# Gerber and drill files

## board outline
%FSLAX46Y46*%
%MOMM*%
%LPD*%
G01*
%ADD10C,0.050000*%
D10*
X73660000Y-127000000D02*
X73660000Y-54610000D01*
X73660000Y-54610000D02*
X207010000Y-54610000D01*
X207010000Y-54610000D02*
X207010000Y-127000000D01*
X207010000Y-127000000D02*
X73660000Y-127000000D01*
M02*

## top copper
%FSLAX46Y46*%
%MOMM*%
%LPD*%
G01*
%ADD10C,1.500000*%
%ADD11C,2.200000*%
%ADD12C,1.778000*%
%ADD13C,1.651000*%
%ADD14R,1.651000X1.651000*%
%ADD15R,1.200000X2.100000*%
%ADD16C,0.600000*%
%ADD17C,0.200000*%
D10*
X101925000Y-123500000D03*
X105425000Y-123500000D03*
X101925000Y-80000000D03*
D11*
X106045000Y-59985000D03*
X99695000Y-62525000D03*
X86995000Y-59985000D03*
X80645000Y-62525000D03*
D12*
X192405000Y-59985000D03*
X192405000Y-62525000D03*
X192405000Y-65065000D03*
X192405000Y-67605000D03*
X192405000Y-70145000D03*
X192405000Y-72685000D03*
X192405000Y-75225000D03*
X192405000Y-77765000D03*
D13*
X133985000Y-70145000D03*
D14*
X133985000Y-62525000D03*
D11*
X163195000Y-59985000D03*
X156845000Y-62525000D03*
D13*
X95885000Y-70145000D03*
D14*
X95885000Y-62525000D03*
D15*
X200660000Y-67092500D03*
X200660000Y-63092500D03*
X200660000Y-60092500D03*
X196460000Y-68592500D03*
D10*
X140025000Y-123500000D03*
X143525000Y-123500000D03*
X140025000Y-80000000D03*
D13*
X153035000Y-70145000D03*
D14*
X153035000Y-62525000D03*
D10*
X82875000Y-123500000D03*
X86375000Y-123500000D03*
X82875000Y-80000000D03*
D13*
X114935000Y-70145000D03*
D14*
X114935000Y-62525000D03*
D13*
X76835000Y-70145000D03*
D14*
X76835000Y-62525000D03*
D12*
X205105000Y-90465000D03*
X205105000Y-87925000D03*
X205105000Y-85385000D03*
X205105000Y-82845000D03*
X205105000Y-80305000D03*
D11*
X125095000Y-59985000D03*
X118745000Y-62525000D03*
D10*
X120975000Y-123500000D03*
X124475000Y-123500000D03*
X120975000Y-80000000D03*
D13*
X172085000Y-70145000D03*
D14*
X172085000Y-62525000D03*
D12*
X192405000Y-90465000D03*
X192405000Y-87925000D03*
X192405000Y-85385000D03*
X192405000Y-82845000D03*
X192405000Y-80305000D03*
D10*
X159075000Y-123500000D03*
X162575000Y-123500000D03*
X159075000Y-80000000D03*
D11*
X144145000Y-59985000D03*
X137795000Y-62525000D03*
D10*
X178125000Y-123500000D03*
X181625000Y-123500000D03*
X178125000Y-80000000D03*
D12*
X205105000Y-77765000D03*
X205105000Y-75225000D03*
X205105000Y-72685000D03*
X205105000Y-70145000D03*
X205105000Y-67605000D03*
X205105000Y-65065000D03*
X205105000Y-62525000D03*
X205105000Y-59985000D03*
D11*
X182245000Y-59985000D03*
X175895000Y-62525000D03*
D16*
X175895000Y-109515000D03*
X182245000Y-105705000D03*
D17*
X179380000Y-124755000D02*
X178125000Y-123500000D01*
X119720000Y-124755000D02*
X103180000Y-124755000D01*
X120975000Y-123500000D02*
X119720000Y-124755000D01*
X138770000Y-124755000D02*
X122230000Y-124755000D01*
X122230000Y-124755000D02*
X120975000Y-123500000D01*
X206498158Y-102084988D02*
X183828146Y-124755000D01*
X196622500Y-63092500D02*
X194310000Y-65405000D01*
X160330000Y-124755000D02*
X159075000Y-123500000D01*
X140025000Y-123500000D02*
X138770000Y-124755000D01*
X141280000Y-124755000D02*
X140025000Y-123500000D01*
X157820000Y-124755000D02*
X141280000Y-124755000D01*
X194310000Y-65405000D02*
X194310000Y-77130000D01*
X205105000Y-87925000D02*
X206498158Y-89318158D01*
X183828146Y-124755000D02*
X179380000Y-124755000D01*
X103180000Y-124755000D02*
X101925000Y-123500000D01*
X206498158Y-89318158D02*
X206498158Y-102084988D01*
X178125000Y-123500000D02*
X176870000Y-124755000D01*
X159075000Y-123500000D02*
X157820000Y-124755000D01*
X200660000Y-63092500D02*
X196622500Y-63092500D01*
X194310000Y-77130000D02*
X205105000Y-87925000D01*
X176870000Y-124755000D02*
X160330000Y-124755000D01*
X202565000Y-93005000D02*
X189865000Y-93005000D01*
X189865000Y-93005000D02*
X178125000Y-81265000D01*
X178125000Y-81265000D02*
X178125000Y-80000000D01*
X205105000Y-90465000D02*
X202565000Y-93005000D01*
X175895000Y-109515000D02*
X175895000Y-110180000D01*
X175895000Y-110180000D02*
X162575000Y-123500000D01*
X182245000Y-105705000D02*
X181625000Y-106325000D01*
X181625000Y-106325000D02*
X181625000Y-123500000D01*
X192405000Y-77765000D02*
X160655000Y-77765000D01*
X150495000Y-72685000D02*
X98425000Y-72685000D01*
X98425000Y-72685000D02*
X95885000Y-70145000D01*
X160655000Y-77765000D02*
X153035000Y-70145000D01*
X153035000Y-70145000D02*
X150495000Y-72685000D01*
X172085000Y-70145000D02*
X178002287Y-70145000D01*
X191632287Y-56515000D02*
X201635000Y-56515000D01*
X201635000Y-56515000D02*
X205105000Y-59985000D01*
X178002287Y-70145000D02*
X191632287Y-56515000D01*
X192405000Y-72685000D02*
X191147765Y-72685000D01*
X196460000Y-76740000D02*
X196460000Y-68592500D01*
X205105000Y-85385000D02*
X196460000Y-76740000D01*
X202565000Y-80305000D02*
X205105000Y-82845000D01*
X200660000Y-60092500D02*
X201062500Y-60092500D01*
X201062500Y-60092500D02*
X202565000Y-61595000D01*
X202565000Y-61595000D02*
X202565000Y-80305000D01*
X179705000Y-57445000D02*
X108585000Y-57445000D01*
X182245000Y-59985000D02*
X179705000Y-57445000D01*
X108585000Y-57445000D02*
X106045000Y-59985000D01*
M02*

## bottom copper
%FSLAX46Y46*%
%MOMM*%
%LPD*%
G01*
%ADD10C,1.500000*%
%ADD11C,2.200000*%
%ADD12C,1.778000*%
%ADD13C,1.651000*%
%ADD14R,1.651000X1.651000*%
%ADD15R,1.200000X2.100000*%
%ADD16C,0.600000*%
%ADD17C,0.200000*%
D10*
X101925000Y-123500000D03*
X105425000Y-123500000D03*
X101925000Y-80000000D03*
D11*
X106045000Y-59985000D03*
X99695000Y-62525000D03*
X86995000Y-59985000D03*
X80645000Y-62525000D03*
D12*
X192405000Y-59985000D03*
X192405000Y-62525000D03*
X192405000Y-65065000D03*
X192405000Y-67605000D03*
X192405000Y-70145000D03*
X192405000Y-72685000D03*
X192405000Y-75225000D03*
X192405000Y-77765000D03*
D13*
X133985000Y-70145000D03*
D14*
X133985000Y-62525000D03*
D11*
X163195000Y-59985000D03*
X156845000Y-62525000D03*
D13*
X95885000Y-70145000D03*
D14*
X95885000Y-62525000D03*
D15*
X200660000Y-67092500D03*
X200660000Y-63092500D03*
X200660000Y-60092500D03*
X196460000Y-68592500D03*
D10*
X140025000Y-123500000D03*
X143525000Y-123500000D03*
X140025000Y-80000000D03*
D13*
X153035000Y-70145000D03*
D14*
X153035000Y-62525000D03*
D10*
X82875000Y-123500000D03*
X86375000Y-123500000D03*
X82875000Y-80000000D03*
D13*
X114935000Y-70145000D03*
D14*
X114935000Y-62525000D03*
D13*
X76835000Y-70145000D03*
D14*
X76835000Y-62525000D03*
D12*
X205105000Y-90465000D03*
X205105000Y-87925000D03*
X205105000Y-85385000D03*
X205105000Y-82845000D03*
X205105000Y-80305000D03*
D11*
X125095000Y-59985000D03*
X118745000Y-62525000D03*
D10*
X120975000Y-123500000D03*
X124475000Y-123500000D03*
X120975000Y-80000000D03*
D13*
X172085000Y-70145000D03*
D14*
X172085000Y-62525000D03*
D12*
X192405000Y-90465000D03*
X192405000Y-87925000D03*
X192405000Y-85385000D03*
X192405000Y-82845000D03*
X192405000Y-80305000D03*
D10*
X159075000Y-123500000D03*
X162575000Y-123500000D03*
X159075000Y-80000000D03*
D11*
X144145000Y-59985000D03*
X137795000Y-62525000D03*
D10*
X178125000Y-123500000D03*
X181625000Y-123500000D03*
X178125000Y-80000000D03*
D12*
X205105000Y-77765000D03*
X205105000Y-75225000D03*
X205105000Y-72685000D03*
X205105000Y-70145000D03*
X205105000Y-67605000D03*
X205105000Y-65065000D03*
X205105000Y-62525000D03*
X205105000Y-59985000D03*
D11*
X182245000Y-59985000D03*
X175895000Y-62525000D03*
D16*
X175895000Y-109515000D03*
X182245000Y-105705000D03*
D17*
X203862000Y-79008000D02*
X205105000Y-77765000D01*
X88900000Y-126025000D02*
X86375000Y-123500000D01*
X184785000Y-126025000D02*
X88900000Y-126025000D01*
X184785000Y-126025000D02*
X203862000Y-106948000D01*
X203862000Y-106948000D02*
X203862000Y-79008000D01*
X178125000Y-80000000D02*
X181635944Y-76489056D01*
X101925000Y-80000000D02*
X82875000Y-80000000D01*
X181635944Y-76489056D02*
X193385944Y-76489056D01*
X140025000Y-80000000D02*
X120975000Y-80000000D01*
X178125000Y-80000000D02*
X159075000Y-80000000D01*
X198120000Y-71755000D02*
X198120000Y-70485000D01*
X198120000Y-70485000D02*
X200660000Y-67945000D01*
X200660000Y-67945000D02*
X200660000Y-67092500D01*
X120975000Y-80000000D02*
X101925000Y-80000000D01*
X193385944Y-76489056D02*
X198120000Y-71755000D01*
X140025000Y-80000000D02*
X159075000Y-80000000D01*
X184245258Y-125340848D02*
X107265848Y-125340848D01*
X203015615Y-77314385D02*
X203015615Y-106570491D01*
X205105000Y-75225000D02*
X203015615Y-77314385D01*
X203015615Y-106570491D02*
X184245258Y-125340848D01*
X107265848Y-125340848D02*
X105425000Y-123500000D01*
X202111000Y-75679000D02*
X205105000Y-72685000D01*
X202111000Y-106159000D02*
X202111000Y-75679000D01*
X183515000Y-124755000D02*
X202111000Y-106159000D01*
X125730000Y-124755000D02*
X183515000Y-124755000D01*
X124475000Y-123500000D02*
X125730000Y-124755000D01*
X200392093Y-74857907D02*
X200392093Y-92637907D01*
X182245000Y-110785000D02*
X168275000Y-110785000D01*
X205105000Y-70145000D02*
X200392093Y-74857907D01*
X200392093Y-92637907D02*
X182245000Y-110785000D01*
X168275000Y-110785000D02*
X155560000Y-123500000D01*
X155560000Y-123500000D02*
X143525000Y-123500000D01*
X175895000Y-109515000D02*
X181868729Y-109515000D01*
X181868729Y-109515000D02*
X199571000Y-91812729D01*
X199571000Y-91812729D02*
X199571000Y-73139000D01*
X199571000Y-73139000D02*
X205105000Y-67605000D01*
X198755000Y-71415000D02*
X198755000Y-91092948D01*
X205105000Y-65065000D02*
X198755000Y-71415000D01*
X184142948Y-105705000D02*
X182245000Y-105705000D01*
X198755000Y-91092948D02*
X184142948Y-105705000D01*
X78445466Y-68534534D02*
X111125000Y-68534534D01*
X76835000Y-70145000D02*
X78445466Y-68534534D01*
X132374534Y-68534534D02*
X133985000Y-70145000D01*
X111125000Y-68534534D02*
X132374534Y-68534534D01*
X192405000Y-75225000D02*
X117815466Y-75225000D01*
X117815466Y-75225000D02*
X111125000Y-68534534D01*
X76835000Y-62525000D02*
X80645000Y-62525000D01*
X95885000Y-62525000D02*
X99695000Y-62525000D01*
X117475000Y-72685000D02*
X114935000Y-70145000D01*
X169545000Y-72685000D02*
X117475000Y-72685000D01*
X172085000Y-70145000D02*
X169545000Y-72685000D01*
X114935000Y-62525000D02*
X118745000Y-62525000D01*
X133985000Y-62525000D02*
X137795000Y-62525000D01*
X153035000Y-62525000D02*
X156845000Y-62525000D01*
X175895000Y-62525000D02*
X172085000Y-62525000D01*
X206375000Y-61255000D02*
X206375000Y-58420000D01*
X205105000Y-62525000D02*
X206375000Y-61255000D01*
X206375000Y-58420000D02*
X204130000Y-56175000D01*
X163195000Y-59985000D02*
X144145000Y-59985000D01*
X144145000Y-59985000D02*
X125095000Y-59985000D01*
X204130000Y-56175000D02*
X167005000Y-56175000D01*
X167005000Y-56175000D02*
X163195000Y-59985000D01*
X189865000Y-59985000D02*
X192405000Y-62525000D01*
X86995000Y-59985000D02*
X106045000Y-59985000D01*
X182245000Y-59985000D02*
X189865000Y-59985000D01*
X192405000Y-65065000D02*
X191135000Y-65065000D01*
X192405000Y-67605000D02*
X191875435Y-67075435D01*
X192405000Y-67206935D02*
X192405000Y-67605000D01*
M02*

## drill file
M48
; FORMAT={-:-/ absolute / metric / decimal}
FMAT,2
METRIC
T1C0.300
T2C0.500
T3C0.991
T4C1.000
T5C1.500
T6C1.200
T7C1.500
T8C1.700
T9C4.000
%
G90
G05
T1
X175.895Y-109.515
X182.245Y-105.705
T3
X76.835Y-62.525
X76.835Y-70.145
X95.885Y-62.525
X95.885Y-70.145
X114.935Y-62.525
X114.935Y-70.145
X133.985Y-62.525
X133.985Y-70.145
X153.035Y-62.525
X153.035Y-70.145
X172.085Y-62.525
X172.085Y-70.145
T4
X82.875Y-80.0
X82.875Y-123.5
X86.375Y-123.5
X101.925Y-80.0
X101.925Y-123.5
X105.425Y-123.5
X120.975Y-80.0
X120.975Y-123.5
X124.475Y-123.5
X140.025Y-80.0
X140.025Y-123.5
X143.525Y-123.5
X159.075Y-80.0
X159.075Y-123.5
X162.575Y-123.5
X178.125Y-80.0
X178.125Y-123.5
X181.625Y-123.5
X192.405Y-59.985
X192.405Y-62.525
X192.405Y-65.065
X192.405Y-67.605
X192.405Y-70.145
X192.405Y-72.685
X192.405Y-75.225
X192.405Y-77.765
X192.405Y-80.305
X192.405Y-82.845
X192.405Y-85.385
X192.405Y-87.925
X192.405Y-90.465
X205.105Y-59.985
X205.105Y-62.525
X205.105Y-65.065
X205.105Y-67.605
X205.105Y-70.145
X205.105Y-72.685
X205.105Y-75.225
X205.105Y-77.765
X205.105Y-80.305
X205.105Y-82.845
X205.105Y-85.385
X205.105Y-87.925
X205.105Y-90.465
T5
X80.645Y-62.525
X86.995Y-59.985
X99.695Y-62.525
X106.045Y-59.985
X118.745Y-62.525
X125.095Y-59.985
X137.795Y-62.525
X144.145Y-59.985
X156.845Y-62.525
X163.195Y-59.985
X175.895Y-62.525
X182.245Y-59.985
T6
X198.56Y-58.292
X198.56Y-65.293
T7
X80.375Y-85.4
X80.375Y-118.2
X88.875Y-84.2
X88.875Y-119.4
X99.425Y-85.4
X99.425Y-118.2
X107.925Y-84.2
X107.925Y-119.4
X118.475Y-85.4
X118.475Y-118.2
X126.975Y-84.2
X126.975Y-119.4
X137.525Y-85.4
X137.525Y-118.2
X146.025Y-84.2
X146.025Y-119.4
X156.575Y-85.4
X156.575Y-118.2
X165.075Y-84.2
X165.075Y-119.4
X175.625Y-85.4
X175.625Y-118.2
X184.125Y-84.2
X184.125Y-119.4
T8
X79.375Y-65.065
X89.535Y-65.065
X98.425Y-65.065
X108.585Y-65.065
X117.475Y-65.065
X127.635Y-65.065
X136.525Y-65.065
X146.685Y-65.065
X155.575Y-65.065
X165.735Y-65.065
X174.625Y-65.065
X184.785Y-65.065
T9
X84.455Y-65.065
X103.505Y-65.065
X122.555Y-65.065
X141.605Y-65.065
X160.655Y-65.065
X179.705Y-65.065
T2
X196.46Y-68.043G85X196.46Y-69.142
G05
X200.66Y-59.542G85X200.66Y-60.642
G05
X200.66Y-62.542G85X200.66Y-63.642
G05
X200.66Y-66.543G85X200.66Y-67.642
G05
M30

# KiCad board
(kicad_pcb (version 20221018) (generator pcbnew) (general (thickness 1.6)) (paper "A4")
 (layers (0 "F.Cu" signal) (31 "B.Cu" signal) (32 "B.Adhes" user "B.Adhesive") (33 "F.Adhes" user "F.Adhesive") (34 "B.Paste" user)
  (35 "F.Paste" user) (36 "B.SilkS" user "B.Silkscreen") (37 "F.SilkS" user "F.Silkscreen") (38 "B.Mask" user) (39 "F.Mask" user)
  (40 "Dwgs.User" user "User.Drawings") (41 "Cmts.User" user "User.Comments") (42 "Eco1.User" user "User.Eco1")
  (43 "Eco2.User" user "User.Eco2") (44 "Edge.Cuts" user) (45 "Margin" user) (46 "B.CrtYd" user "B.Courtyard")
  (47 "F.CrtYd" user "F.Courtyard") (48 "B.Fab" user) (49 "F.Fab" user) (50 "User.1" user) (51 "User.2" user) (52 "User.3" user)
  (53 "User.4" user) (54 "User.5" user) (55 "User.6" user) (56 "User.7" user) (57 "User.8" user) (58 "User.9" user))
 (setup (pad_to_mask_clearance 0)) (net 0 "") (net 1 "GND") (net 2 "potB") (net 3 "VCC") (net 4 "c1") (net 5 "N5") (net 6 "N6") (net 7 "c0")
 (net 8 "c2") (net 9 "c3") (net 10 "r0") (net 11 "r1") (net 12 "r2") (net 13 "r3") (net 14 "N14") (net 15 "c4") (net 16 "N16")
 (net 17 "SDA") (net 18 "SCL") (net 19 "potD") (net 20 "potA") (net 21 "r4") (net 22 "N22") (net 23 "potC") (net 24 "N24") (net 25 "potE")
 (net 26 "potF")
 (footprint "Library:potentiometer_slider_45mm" (layer "F.Cu") (at 110.625 124.3 90)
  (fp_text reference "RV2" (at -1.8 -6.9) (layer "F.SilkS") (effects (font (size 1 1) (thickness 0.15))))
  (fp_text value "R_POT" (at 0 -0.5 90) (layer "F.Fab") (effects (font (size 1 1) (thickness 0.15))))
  (pad "" np_thru_hole circle (at 4.9 -2.7 90) (size 1.5 1.5) (drill 1.5) (layers "*.Cu" "*.Mask"))
  (pad "" np_thru_hole circle (at 6.1 -11.2 90) (size 1.5 1.5) (drill 1.5) (layers "*.Cu" "*.Mask"))
  (pad "" np_thru_hole circle (at 38.9 -11.2 90) (size 1.5 1.5) (drill 1.5) (layers "*.Cu" "*.Mask"))
  (pad "" np_thru_hole circle (at 40.1 -2.7 90) (size 1.5 1.5) (drill 1.5) (layers "*.Cu" "*.Mask"))
  (pad "1" thru_hole circle (at 0.8 -8.7 90) (size 1.5 1.5) (drill 1) (layers "*.Cu" "*.Mask") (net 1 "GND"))
  (pad "2" thru_hole circle (at 0.8 -5.2 90) (size 1.5 1.5) (drill 1) (layers "*.Cu" "*.Mask") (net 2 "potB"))
  (pad "3" thru_hole circle (at 44.3 -8.7 90) (size 1.5 1.5) (drill 1) (layers "*.Cu" "*.Mask") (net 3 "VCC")))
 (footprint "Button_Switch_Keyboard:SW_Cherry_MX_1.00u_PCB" (layer "F.Cu") (at 106.045 59.985)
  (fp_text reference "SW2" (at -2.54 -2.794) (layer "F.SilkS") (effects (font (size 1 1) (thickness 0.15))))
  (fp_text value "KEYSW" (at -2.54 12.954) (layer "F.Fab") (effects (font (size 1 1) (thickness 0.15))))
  (pad "" np_thru_hole circle (at -7.62 5.08) (size 1.7 1.7) (drill 1.7) (layers "*.Cu" "*.Mask"))
  (pad "" np_thru_hole circle (at -2.54 5.08) (size 4 4) (drill 4) (layers "*.Cu" "*.Mask"))
  (pad "" np_thru_hole circle (at 2.54 5.08) (size 1.7 1.7) (drill 1.7) (layers "*.Cu" "*.Mask"))
  (pad "1" thru_hole circle (at 0 0) (size 2.2 2.2) (drill 1.5) (layers "*.Cu" "*.Mask") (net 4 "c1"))
  (pad "2" thru_hole circle (at -6.35 2.54) (size 2.2 2.2) (drill 1.5) (layers "*.Cu" "*.Mask") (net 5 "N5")))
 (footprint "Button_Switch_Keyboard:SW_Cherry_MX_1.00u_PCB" (layer "F.Cu") (at 86.995 59.985)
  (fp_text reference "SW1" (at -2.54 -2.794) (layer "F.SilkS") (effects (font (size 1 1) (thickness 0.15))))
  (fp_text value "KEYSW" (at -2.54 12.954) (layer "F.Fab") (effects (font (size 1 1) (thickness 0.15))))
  (pad "" np_thru_hole circle (at -7.62 5.08) (size 1.7 1.7) (drill 1.7) (layers "*.Cu" "*.Mask"))
  (pad "" np_thru_hole circle (at -2.54 5.08) (size 4 4) (drill 4) (layers "*.Cu" "*.Mask"))
  (pad "" np_thru_hole circle (at 2.54 5.08) (size 1.7 1.7) (drill 1.7) (layers "*.Cu" "*.Mask"))
  (pad "1" thru_hole circle (at 0 0) (size 2.2 2.2) (drill 1.5) (layers "*.Cu" "*.Mask") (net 4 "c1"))
  (pad "2" thru_hole circle (at -6.35 2.54) (size 2.2 2.2) (drill 1.5) (layers "*.Cu" "*.Mask") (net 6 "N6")))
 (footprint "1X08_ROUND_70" (layer "F.Cu") (at 192.405 68.875 -90)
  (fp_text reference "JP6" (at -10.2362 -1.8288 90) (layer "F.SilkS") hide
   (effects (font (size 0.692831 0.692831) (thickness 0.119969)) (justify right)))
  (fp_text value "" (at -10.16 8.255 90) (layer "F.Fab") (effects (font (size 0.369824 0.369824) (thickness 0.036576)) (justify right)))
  (pad "1" thru_hole circle (at -8.89 0) (size 1.778 1.778) (drill 1) (layers "*.Cu" "*.Mask") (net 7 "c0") (solder_mask_margin 0.0508))
  (pad "2" thru_hole circle (at -6.35 0) (size 1.778 1.778) (drill 1) (layers "*.Cu" "*.Mask") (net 4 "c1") (solder_mask_margin 0.0508))
  (pad "3" thru_hole circle (at -3.81 0) (size 1.778 1.778) (drill 1) (layers "*.Cu" "*.Mask") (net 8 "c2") (solder_mask_margin 0.0508))
  (pad "4" thru_hole circle (at -1.27 0) (size 1.778 1.778) (drill 1) (layers "*.Cu" "*.Mask") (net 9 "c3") (solder_mask_margin 0.0508))
  (pad "5" thru_hole circle (at 1.27 0) (size 1.778 1.778) (drill 1) (layers "*.Cu" "*.Mask") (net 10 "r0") (solder_mask_margin 0.0508))
  (pad "6" thru_hole circle (at 3.81 0) (size 1.778 1.778) (drill 1) (layers "*.Cu" "*.Mask") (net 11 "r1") (solder_mask_margin 0.0508))
  (pad "7" thru_hole circle (at 6.35 0) (size 1.778 1.778) (drill 1) (layers "*.Cu" "*.Mask") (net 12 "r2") (solder_mask_margin 0.0508))
  (pad "8" thru_hole circle (at 8.89 0) (size 1.778 1.778) (drill 1) (layers "*.Cu" "*.Mask") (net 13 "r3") (solder_mask_margin 0.0508)))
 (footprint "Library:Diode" (layer "F.Cu") (at 133.985 66.335 90)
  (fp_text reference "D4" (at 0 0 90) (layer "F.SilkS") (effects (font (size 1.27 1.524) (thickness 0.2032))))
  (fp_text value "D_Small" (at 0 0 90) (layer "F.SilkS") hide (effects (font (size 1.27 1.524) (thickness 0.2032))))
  (pad "1" thru_hole circle (at -3.81 0 90) (size 1.651 1.651) (drill 0.9906) (layers "*.Cu" "*.SilkS" "*.Mask") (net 12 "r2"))
  (pad "2" thru_hole rect (at 3.81 0 90) (size 1.651 1.651) (drill 0.9906) (layers "*.Cu" "*.SilkS" "*.Mask") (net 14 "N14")))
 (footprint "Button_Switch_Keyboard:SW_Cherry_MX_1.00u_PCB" (layer "F.Cu") (at 163.195 59.985)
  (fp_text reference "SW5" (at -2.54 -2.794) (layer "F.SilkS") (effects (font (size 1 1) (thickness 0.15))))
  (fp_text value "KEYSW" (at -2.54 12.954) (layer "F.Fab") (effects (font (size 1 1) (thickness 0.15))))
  (pad "" np_thru_hole circle (at -7.62 5.08) (size 1.7 1.7) (drill 1.7) (layers "*.Cu" "*.Mask"))
  (pad "" np_thru_hole circle (at -2.54 5.08) (size 4 4) (drill 4) (layers "*.Cu" "*.Mask"))
  (pad "" np_thru_hole circle (at 2.54 5.08) (size 1.7 1.7) (drill 1.7) (layers "*.Cu" "*.Mask"))
  (pad "1" thru_hole circle (at 0 0) (size 2.2 2.2) (drill 1.5) (layers "*.Cu" "*.Mask") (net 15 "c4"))
  (pad "2" thru_hole circle (at -6.35 2.54) (size 2.2 2.2) (drill 1.5) (layers "*.Cu" "*.Mask") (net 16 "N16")))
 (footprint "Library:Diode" (layer "F.Cu") (at 95.885 66.335 90)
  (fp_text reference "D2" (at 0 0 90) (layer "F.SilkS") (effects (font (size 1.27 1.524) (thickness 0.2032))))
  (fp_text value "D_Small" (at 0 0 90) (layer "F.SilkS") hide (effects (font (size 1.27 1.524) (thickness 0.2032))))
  (pad "1" thru_hole circle (at -3.81 0 90) (size 1.651 1.651) (drill 0.9906) (layers "*.Cu" "*.SilkS" "*.Mask") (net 13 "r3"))
  (pad "2" thru_hole rect (at 3.81 0 90) (size 1.651 1.651) (drill 0.9906) (layers "*.Cu" "*.SilkS" "*.Mask") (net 5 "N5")))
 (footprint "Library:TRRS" (layer "F.Cu") (at 198.56 56.7925)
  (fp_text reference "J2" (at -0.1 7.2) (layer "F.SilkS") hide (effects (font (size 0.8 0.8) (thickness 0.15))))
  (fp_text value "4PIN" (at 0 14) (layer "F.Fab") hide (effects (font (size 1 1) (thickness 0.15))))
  (pad "" np_thru_hole circle (at 0 1.5) (size 1.2 1.2) (drill 1.2) (layers "*.Cu" "*.Mask" "F.SilkS"))
  (pad "" np_thru_hole circle (at 0 8.5) (size 1.2 1.2) (drill 1.2) (layers "*.Cu" "*.Mask" "F.SilkS"))
  (pad "1" thru_hole rect (at 2.1 10.3) (size 1.2 2.1) (drill oval 0.5 1.6) (layers "*.Cu" "*.Mask" "F.SilkS") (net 3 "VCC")
   (clearance 0.15))
  (pad "2" thru_hole rect (at 2.1 6.3) (size 1.2 2.1) (drill oval 0.5 1.6) (layers "*.Cu" "*.Mask" "F.SilkS") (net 1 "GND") (clearance 0.15))
  (pad "3" thru_hole rect (at 2.1 3.3) (size 1.2 2.1) (drill oval 0.5 1.6) (layers "*.Cu" "*.Mask" "F.SilkS") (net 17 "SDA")
   (clearance 0.15))
  (pad "4" thru_hole rect (at -2.1 11.8) (size 1.2 2.1) (drill oval 0.5 1.6) (layers "*.Cu" "*.Mask" "F.SilkS") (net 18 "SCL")
   (clearance 0.15)))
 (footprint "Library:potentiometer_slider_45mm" (layer "F.Cu") (at 148.725 124.3 90)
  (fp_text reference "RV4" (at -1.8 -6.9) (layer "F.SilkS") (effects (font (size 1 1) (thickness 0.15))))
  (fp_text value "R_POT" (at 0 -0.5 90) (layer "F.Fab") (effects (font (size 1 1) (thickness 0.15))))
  (pad "" np_thru_hole circle (at 4.9 -2.7 90) (size 1.5 1.5) (drill 1.5) (layers "*.Cu" "*.Mask"))
  (pad "" np_thru_hole circle (at 6.1 -11.2 90) (size 1.5 1.5) (drill 1.5) (layers "*.Cu" "*.Mask"))
  (pad "" np_thru_hole circle (at 38.9 -11.2 90) (size 1.5 1.5) (drill 1.5) (layers "*.Cu" "*.Mask"))
  (pad "" np_thru_hole circle (at 40.1 -2.7 90) (size 1.5 1.5) (drill 1.5) (layers "*.Cu" "*.Mask"))
  (pad "1" thru_hole circle (at 0.8 -8.7 90) (size 1.5 1.5) (drill 1) (layers "*.Cu" "*.Mask") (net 1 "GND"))
  (pad "2" thru_hole circle (at 0.8 -5.2 90) (size 1.5 1.5) (drill 1) (layers "*.Cu" "*.Mask") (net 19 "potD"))
  (pad "3" thru_hole circle (at 44.3 -8.7 90) (size 1.5 1.5) (drill 1) (layers "*.Cu" "*.Mask") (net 3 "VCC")))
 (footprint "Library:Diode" (layer "F.Cu") (at 153.035 66.335 90)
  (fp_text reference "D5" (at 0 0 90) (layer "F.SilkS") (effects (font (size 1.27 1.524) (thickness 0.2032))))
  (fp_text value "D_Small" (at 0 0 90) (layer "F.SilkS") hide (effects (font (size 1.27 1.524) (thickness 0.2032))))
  (pad "1" thru_hole circle (at -3.81 0 90) (size 1.651 1.651) (drill 0.9906) (layers "*.Cu" "*.SilkS" "*.Mask") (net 13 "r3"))
  (pad "2" thru_hole rect (at 3.81 0 90) (size 1.651 1.651) (drill 0.9906) (layers "*.Cu" "*.SilkS" "*.Mask") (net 16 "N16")))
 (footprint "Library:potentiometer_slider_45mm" (layer "F.Cu") (at 91.575 124.3 90)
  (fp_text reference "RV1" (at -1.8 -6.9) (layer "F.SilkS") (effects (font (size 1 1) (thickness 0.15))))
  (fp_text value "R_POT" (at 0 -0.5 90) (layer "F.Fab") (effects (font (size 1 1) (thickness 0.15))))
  (pad "" np_thru_hole circle (at 4.9 -2.7 90) (size 1.5 1.5) (drill 1.5) (layers "*.Cu" "*.Mask"))
  (pad "" np_thru_hole circle (at 6.1 -11.2 90) (size 1.5 1.5) (drill 1.5) (layers "*.Cu" "*.Mask"))
  (pad "" np_thru_hole circle (at 38.9 -11.2 90) (size 1.5 1.5) (drill 1.5) (layers "*.Cu" "*.Mask"))
  (pad "" np_thru_hole circle (at 40.1 -2.7 90) (size 1.5 1.5) (drill 1.5) (layers "*.Cu" "*.Mask"))
  (pad "1" thru_hole circle (at 0.8 -8.7 90) (size 1.5 1.5) (drill 1) (layers "*.Cu" "*.Mask") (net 1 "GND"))
  (pad "2" thru_hole circle (at 0.8 -5.2 90) (size 1.5 1.5) (drill 1) (layers "*.Cu" "*.Mask") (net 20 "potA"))
  (pad "3" thru_hole circle (at 44.3 -8.7 90) (size 1.5 1.5) (drill 1) (layers "*.Cu" "*.Mask") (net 3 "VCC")))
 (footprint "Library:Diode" (layer "F.Cu") (at 114.935 66.335 90)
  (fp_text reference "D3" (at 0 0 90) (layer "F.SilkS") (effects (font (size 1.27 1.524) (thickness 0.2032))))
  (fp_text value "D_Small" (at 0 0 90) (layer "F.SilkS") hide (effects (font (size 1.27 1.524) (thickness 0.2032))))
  (pad "1" thru_hole circle (at -3.81 0 90) (size 1.651 1.651) (drill 0.9906) (layers "*.Cu" "*.SilkS" "*.Mask") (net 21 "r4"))
  (pad "2" thru_hole rect (at 3.81 0 90) (size 1.651 1.651) (drill 0.9906) (layers "*.Cu" "*.SilkS" "*.Mask") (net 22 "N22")))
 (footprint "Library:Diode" (layer "F.Cu") (at 76.835 66.335 90)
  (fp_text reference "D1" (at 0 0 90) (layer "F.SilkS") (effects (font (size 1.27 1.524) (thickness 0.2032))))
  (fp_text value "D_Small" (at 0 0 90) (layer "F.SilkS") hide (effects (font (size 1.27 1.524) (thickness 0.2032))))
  (pad "1" thru_hole circle (at -3.81 0 90) (size 1.651 1.651) (drill 0.9906) (layers "*.Cu" "*.SilkS" "*.Mask") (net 12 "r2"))
  (pad "2" thru_hole rect (at 3.81 0 90) (size 1.651 1.651) (drill 0.9906) (layers "*.Cu" "*.SilkS" "*.Mask") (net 6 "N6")))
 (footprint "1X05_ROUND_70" (layer "F.Cu") (at 205.105 85.385 90)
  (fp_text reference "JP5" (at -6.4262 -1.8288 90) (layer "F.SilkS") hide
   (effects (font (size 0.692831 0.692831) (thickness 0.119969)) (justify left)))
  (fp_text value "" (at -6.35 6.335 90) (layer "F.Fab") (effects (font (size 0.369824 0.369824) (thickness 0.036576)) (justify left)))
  (pad "1" thru_hole circle (at -5.08 0 180) (size 1.778 1.778) (drill 1) (layers "*.Cu" "*.Mask") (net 3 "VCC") (solder_mask_margin 0.0508))
  (pad "2" thru_hole circle (at -2.54 0 180) (size 1.778 1.778) (drill 1) (layers "*.Cu" "*.Mask") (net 1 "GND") (solder_mask_margin 0.0508))
  (pad "3" thru_hole circle (at 0 0 180) (size 1.778 1.778) (drill 1) (layers "*.Cu" "*.Mask") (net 18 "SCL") (solder_mask_margin 0.0508))
  (pad "4" thru_hole circle (at 2.54 0 180) (size 1.778 1.778) (drill 1) (layers "*.Cu" "*.Mask") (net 17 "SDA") (solder_mask_margin 0.0508))
  (pad "5" thru_hole circle (at 5.08 0 180) (size 1.778 1.778) (drill 1) (layers "*.Cu" "*.Mask") (solder_mask_margin 0.0508)))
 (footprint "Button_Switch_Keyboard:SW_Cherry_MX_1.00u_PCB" (layer "F.Cu") (at 125.095 59.985)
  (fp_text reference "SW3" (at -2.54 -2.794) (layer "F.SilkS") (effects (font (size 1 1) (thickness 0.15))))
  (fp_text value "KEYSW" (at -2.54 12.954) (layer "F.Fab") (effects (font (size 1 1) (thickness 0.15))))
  (pad "" np_thru_hole circle (at -7.62 5.08) (size 1.7 1.7) (drill 1.7) (layers "*.Cu" "*.Mask"))
  (pad "" np_thru_hole circle (at -2.54 5.08) (size 4 4) (drill 4) (layers "*.Cu" "*.Mask"))
  (pad "" np_thru_hole circle (at 2.54 5.08) (size 1.7 1.7) (drill 1.7) (layers "*.Cu" "*.Mask"))
  (pad "1" thru_hole circle (at 0 0) (size 2.2 2.2) (drill 1.5) (layers "*.Cu" "*.Mask") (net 15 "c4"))
  (pad "2" thru_hole circle (at -6.35 2.54) (size 2.2 2.2) (drill 1.5) (layers "*.Cu" "*.Mask") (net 22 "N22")))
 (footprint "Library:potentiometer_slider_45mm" (layer "F.Cu") (at 129.675 124.3 90)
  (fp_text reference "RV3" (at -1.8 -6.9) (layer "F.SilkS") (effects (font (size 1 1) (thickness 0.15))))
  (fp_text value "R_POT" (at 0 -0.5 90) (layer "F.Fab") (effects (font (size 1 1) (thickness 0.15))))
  (pad "" np_thru_hole circle (at 4.9 -2.7 90) (size 1.5 1.5) (drill 1.5) (layers "*.Cu" "*.Mask"))
  (pad "" np_thru_hole circle (at 6.1 -11.2 90) (size 1.5 1.5) (drill 1.5) (layers "*.Cu" "*.Mask"))
  (pad "" np_thru_hole circle (at 38.9 -11.2 90) (size 1.5 1.5) (drill 1.5) (layers "*.Cu" "*.Mask"))
  (pad "" np_thru_hole circle (at 40.1 -2.7 90) (size 1.5 1.5) (drill 1.5) (layers "*.Cu" "*.Mask"))
  (pad "1" thru_hole circle (at 0.8 -8.7 90) (size 1.5 1.5) (drill 1) (layers "*.Cu" "*.Mask") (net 1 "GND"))
  (pad "2" thru_hole circle (at 0.8 -5.2 90) (size 1.5 1.5) (drill 1) (layers "*.Cu" "*.Mask") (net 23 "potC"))
  (pad "3" thru_hole circle (at 44.3 -8.7 90) (size 1.5 1.5) (drill 1) (layers "*.Cu" "*.Mask") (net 3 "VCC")))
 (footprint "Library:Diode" (layer "F.Cu") (at 172.085 66.335 90)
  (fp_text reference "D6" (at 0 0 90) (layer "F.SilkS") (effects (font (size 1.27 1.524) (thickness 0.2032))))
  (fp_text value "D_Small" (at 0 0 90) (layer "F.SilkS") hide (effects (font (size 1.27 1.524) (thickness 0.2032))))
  (pad "1" thru_hole circle (at -3.81 0 90) (size 1.651 1.651) (drill 0.9906) (layers "*.Cu" "*.SilkS" "*.Mask") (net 21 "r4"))
  (pad "2" thru_hole rect (at 3.81 0 90) (size 1.651 1.651) (drill 0.9906) (layers "*.Cu" "*.SilkS" "*.Mask") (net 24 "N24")))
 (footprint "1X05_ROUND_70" (layer "F.Cu") (at 192.405 85.385 90)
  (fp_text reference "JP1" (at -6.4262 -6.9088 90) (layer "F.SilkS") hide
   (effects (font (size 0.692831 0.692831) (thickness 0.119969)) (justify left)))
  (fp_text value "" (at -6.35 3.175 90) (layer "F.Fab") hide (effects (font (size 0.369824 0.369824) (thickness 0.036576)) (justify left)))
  (pad "1" thru_hole circle (at -5.08 0 180) (size 1.778 1.778) (drill 1) (layers "*.Cu" "*.Mask") (solder_mask_margin 0.0508))
  (pad "2" thru_hole circle (at -2.54 0 180) (size 1.778 1.778) (drill 1) (layers "*.Cu" "*.Mask") (solder_mask_margin 0.0508))
  (pad "3" thru_hole circle (at 0 0 180) (size 1.778 1.778) (drill 1) (layers "*.Cu" "*.Mask") (solder_mask_margin 0.0508))
  (pad "4" thru_hole circle (at 2.54 0 180) (size 1.778 1.778) (drill 1) (layers "*.Cu" "*.Mask") (solder_mask_margin 0.0508))
  (pad "5" thru_hole circle (at 5.08 0 180) (size 1.778 1.778) (drill 1) (layers "*.Cu" "*.Mask") (solder_mask_margin 0.0508)))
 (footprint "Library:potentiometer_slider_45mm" (layer "F.Cu") (at 167.775 124.3 90)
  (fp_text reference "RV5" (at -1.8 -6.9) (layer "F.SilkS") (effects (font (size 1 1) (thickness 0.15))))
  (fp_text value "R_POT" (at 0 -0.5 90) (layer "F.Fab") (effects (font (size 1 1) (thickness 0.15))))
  (pad "" np_thru_hole circle (at 4.9 -2.7 90) (size 1.5 1.5) (drill 1.5) (layers "*.Cu" "*.Mask"))
  (pad "" np_thru_hole circle (at 6.1 -11.2 90) (size 1.5 1.5) (drill 1.5) (layers "*.Cu" "*.Mask"))
  (pad "" np_thru_hole circle (at 38.9 -11.2 90) (size 1.5 1.5) (drill 1.5) (layers "*.Cu" "*.Mask"))
  (pad "" np_thru_hole circle (at 40.1 -2.7 90) (size 1.5 1.5) (drill 1.5) (layers "*.Cu" "*.Mask"))
  (pad "1" thru_hole circle (at 0.8 -8.7 90) (size 1.5 1.5) (drill 1) (layers "*.Cu" "*.Mask") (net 1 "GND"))
  (pad "2" thru_hole circle (at 0.8 -5.2 90) (size 1.5 1.5) (drill 1) (layers "*.Cu" "*.Mask") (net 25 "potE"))
  (pad "3" thru_hole circle (at 44.3 -8.7 90) (size 1.5 1.5) (drill 1) (layers "*.Cu" "*.Mask") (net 3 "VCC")))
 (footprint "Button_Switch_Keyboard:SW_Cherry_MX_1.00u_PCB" (layer "F.Cu") (at 144.145 59.985)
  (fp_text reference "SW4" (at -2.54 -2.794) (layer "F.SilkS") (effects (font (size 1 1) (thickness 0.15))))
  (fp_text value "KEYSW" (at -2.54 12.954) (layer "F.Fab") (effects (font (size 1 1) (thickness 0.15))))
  (pad "" np_thru_hole circle (at -7.62 5.08) (size 1.7 1.7) (drill 1.7) (layers "*.Cu" "*.Mask"))
  (pad "" np_thru_hole circle (at -2.54 5.08) (size 4 4) (drill 4) (layers "*.Cu" "*.Mask"))
  (pad "" np_thru_hole circle (at 2.54 5.08) (size 1.7 1.7) (drill 1.7) (layers "*.Cu" "*.Mask"))
  (pad "1" thru_hole circle (at 0 0) (size 2.2 2.2) (drill 1.5) (layers "*.Cu" "*.Mask") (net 15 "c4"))
  (pad "2" thru_hole circle (at -6.35 2.54) (size 2.2 2.2) (drill 1.5) (layers "*.Cu" "*.Mask") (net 14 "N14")))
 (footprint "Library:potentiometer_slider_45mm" (layer "F.Cu") (at 186.825 124.3 90)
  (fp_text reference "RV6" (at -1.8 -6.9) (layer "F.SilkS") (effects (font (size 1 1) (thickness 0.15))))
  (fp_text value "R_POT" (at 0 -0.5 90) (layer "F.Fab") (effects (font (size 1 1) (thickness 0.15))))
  (pad "" np_thru_hole circle (at 4.9 -2.7 90) (size 1.5 1.5) (drill 1.5) (layers "*.Cu" "*.Mask"))
  (pad "" np_thru_hole circle (at 6.1 -11.2 90) (size 1.5 1.5) (drill 1.5) (layers "*.Cu" "*.Mask"))
  (pad "" np_thru_hole circle (at 38.9 -11.2 90) (size 1.5 1.5) (drill 1.5) (layers "*.Cu" "*.Mask"))
  (pad "" np_thru_hole circle (at 40.1 -2.7 90) (size 1.5 1.5) (drill 1.5) (layers "*.Cu" "*.Mask"))
  (pad "1" thru_hole circle (at 0.8 -8.7 90) (size 1.5 1.5) (drill 1) (layers "*.Cu" "*.Mask") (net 1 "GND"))
  (pad "2" thru_hole circle (at 0.8 -5.2 90) (size 1.5 1.5) (drill 1) (layers "*.Cu" "*.Mask") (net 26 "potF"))
  (pad "3" thru_hole circle (at 44.3 -8.7 90) (size 1.5 1.5) (drill 1) (layers "*.Cu" "*.Mask") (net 3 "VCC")))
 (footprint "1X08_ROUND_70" (layer "F.Cu") (at 205.105 68.875 90)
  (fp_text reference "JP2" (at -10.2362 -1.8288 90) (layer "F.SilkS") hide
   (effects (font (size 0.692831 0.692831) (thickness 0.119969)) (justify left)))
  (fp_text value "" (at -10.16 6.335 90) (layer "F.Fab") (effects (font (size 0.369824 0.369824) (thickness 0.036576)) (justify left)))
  (pad "1" thru_hole circle (at -8.89 0 180) (size 1.778 1.778) (drill 1) (layers "*.Cu" "*.Mask") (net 20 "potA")
   (solder_mask_margin 0.0508))
  (pad "2" thru_hole circle (at -6.35 0 180) (size 1.778 1.778) (drill 1) (layers "*.Cu" "*.Mask") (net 2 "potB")
   (solder_mask_margin 0.0508))
  (pad "3" thru_hole circle (at -3.81 0 180) (size 1.778 1.778) (drill 1) (layers "*.Cu" "*.Mask") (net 23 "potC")
   (solder_mask_margin 0.0508))
  (pad "4" thru_hole circle (at -1.27 0 180) (size 1.778 1.778) (drill 1) (layers "*.Cu" "*.Mask") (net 19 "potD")
   (solder_mask_margin 0.0508))
  (pad "5" thru_hole circle (at 1.27 0 180) (size 1.778 1.778) (drill 1) (layers "*.Cu" "*.Mask") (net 25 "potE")
   (solder_mask_margin 0.0508))
  (pad "6" thru_hole circle (at 3.81 0 180) (size 1.778 1.778) (drill 1) (layers "*.Cu" "*.Mask") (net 26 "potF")
   (solder_mask_margin 0.0508))
  (pad "7" thru_hole circle (at 6.35 0 180) (size 1.778 1.778) (drill 1) (layers "*.Cu" "*.Mask") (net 15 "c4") (solder_mask_margin 0.0508))
  (pad "8" thru_hole circle (at 8.89 0 180) (size 1.778 1.778) (drill 1) (layers "*.Cu" "*.Mask") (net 21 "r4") (solder_mask_margin 0.0508)))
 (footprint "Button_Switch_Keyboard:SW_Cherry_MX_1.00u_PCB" (layer "F.Cu") (at 182.245 59.985)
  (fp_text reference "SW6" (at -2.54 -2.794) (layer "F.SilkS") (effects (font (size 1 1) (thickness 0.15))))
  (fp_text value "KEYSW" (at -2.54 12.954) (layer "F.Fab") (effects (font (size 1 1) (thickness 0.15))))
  (pad "" np_thru_hole circle (at -7.62 5.08) (size 1.7 1.7) (drill 1.7) (layers "*.Cu" "*.Mask"))
  (pad "" np_thru_hole circle (at -2.54 5.08) (size 4 4) (drill 4) (layers "*.Cu" "*.Mask"))
  (pad "" np_thru_hole circle (at 2.54 5.08) (size 1.7 1.7) (drill 1.7) (layers "*.Cu" "*.Mask"))
  (pad "1" thru_hole circle (at 0 0) (size 2.2 2.2) (drill 1.5) (layers "*.Cu" "*.Mask") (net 4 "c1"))
  (pad "2" thru_hole circle (at -6.35 2.54) (size 2.2 2.2) (drill 1.5) (layers "*.Cu" "*.Mask") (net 24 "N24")))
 (gr_line (start 73.66 127) (end 73.66 54.61) (stroke (width 0.05) (type default)) (layer "Edge.Cuts"))
 (gr_line (start 73.66 54.61) (end 207.01 54.61) (stroke (width 0.05) (type default)) (layer "Edge.Cuts"))
 (gr_line (start 207.01 54.61) (end 207.01 127) (stroke (width 0.05) (type default)) (layer "Edge.Cuts"))
 (gr_line (start 207.01 127) (end 73.66 127) (stroke (width 0.05) (type default)) (layer "Edge.Cuts"))
 (segment (start 179.38 124.755) (end 178.125 123.5) (width 0.2) (layer "F.Cu") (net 1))
 (segment (start 119.72 124.755) (end 103.18 124.755) (width 0.2) (layer "F.Cu") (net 1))
 (segment (start 120.975 123.5) (end 119.72 124.755) (width 0.2) (layer "F.Cu") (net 1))
 (segment (start 138.77 124.755) (end 122.23 124.755) (width 0.2) (layer "F.Cu") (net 1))
 (segment (start 122.23 124.755) (end 120.975 123.5) (width 0.2) (layer "F.Cu") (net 1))
 (segment (start 206.498158 102.084988) (end 183.828146 124.755) (width 0.2) (layer "F.Cu") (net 1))
 (segment (start 196.6225 63.0925) (end 194.31 65.405) (width 0.2) (layer "F.Cu") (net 1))
 (segment (start 160.33 124.755) (end 159.075 123.5) (width 0.2) (layer "F.Cu") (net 1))
 (segment (start 140.025 123.5) (end 138.77 124.755) (width 0.2) (layer "F.Cu") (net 1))
 (segment (start 141.28 124.755) (end 140.025 123.5) (width 0.2) (layer "F.Cu") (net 1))
 (segment (start 157.82 124.755) (end 141.28 124.755) (width 0.2) (layer "F.Cu") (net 1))
 (segment (start 194.31 65.405) (end 194.31 77.13) (width 0.2) (layer "F.Cu") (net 1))
 (segment (start 205.105 87.925) (end 206.498158 89.318158) (width 0.2) (layer "F.Cu") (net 1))
 (segment (start 183.828146 124.755) (end 179.38 124.755) (width 0.2) (layer "F.Cu") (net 1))
 (segment (start 103.18 124.755) (end 101.925 123.5) (width 0.2) (layer "F.Cu") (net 1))
 (segment (start 206.498158 89.318158) (end 206.498158 102.084988) (width 0.2) (layer "F.Cu") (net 1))
 (segment (start 178.125 123.5) (end 176.87 124.755) (width 0.2) (layer "F.Cu") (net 1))
 (segment (start 159.075 123.5) (end 157.82 124.755) (width 0.2) (layer "F.Cu") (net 1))
 (segment (start 200.66 63.0925) (end 196.6225 63.0925) (width 0.2) (layer "F.Cu") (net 1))
 (segment (start 194.31 77.13) (end 205.105 87.925) (width 0.2) (layer "F.Cu") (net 1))
 (segment (start 176.87 124.755) (end 160.33 124.755) (width 0.2) (layer "F.Cu") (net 1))
 (segment (start 203.862 79.008) (end 205.105 77.765) (width 0.2) (layer "B.Cu") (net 20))
 (segment (start 88.9 126.025) (end 86.375 123.5) (width 0.2) (layer "B.Cu") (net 20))
 (segment (start 184.785 126.025) (end 88.9 126.025) (width 0.2) (layer "B.Cu") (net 20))
 (segment (start 184.785 126.025) (end 203.862 106.948) (width 0.2) (layer "B.Cu") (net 20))
 (segment (start 203.862 106.948) (end 203.862 79.008) (width 0.2) (layer "B.Cu") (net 20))
 (segment (start 202.565 93.005) (end 189.865 93.005) (width 0.2) (layer "F.Cu") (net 3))
 (segment (start 189.865 93.005) (end 178.125 81.265) (width 0.2) (layer "F.Cu") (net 3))
 (segment (start 178.125 81.265) (end 178.125 80) (width 0.2) (layer "F.Cu") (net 3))
 (segment (start 205.105 90.465) (end 202.565 93.005) (width 0.2) (layer "F.Cu") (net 3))
 (segment (start 178.125 80) (end 181.635944 76.489056) (width 0.2) (layer "B.Cu") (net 3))
 (segment (start 101.925 80) (end 82.875 80) (width 0.2) (layer "B.Cu") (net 3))
 (segment (start 181.635944 76.489056) (end 193.385944 76.489056) (width 0.2) (layer "B.Cu") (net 3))
 (segment (start 140.025 80) (end 120.975 80) (width 0.2) (layer "B.Cu") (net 3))
 (segment (start 178.125 80) (end 159.075 80) (width 0.2) (layer "B.Cu") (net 3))
 (segment (start 198.12 71.755) (end 198.12 70.485) (width 0.2) (layer "B.Cu") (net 3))
 (segment (start 198.12 70.485) (end 200.66 67.945) (width 0.2) (layer "B.Cu") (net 3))
 (segment (start 200.66 67.945) (end 200.66 67.0925) (width 0.2) (layer "B.Cu") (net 3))
 (segment (start 120.975 80) (end 101.925 80) (width 0.2) (layer "B.Cu") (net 3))
 (segment (start 193.385944 76.489056) (end 198.12 71.755) (width 0.2) (layer "B.Cu") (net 3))
 (segment (start 140.025 80) (end 159.075 80) (width 0.2) (layer "B.Cu") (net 3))
 (segment (start 184.245258 125.340848) (end 107.265848 125.340848) (width 0.2) (layer "B.Cu") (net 2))
 (segment (start 203.015615 77.314385) (end 203.015615 106.570491) (width 0.2) (layer "B.Cu") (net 2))
 (segment (start 205.105 75.225) (end 203.015615 77.314385) (width 0.2) (layer "B.Cu") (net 2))
 (segment (start 203.015615 106.570491) (end 184.245258 125.340848) (width 0.2) (layer "B.Cu") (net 2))
 (segment (start 107.265848 125.340848) (end 105.425 123.5) (width 0.2) (layer "B.Cu") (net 2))
 (segment (start 202.111 75.679) (end 205.105 72.685) (width 0.2) (layer "B.Cu") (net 23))
 (segment (start 202.111 106.159) (end 202.111 75.679) (width 0.2) (layer "B.Cu") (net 23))
 (segment (start 183.515 124.755) (end 202.111 106.159) (width 0.2) (layer "B.Cu") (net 23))
 (segment (start 125.73 124.755) (end 183.515 124.755) (width 0.2) (layer "B.Cu") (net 23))
 (segment (start 124.475 123.5) (end 125.73 124.755) (width 0.2) (layer "B.Cu") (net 23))
 (segment (start 200.392093 74.857907) (end 200.392093 92.637907) (width 0.2) (layer "B.Cu") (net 19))
 (segment (start 182.245 110.785) (end 168.275 110.785) (width 0.2) (layer "B.Cu") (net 19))
 (segment (start 205.105 70.145) (end 200.392093 74.857907) (width 0.2) (layer "B.Cu") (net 19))
 (segment (start 200.392093 92.637907) (end 182.245 110.785) (width 0.2) (layer "B.Cu") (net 19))
 (segment (start 168.275 110.785) (end 155.56 123.5) (width 0.2) (layer "B.Cu") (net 19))
 (segment (start 155.56 123.5) (end 143.525 123.5) (width 0.2) (layer "B.Cu") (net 19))
 (segment (start 175.895 109.515) (end 175.895 110.18) (width 0.2) (layer "F.Cu") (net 25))
 (segment (start 175.895 110.18) (end 162.575 123.5) (width 0.2) (layer "F.Cu") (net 25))
 (via (at 175.895 109.515) (size 0.6) (drill 0.3) (layers "F.Cu" "B.Cu") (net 25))
 (segment (start 175.895 109.515) (end 181.868729 109.515) (width 0.2) (layer "B.Cu") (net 25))
 (segment (start 181.868729 109.515) (end 199.571 91.812729) (width 0.2) (layer "B.Cu") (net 25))
 (segment (start 199.571 91.812729) (end 199.571 73.139) (width 0.2) (layer "B.Cu") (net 25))
 (segment (start 199.571 73.139) (end 205.105 67.605) (width 0.2) (layer "B.Cu") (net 25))
 (segment (start 182.245 105.705) (end 181.625 106.325) (width 0.2) (layer "F.Cu") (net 26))
 (segment (start 181.625 106.325) (end 181.625 123.5) (width 0.2) (layer "F.Cu") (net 26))
 (via (at 182.245 105.705) (size 0.6) (drill 0.3) (layers "F.Cu" "B.Cu") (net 26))
 (segment (start 198.755 71.415) (end 198.755 91.092948) (width 0.2) (layer "B.Cu") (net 26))
 (segment (start 205.105 65.065) (end 198.755 71.415) (width 0.2) (layer "B.Cu") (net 26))
 (segment (start 184.142948 105.705) (end 182.245 105.705) (width 0.2) (layer "B.Cu") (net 26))
 (segment (start 198.755 91.092948) (end 184.142948 105.705) (width 0.2) (layer "B.Cu") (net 26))
 (segment (start 78.445466 68.534534) (end 111.125 68.534534) (width 0.2) (layer "B.Cu") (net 12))
 (segment (start 76.835 70.145) (end 78.445466 68.534534) (width 0.2) (layer "B.Cu") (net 12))
 (segment (start 132.374534 68.534534) (end 133.985 70.145) (width 0.2) (layer "B.Cu") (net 12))
 (segment (start 111.125 68.534534) (end 132.374534 68.534534) (width 0.2) (layer "B.Cu") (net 12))
 (segment (start 192.405 75.225) (end 117.815466 75.225) (width 0.2) (layer "B.Cu") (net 12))
 (segment (start 117.815466 75.225) (end 111.125 68.534534) (width 0.2) (layer "B.Cu") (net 12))
 (segment (start 76.835 62.525) (end 80.645 62.525) (width 0.2) (layer "B.Cu") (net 6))
 (segment (start 192.405 77.765) (end 160.655 77.765) (width 0.2) (layer "F.Cu") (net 13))
 (segment (start 150.495 72.685) (end 98.425 72.685) (width 0.2) (layer "F.Cu") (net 13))
 (segment (start 98.425 72.685) (end 95.885 70.145) (width 0.2) (layer "F.Cu") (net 13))
 (segment (start 160.655 77.765) (end 153.035 70.145) (width 0.2) (layer "F.Cu") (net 13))
 (segment (start 153.035 70.145) (end 150.495 72.685) (width 0.2) (layer "F.Cu") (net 13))
 (segment (start 95.885 62.525) (end 99.695 62.525) (width 0.2) (layer "B.Cu") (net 5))
 (segment (start 172.085 70.145) (end 178.002287 70.145) (width 0.2) (layer "F.Cu") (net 21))
 (segment (start 191.632287 56.515) (end 201.635 56.515) (width 0.2) (layer "F.Cu") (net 21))
 (segment (start 201.635 56.515) (end 205.105 59.985) (width 0.2) (layer "F.Cu") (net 21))
 (segment (start 178.002287 70.145) (end 191.632287 56.515) (width 0.2) (layer "F.Cu") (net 21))
 (segment (start 117.475 72.685) (end 114.935 70.145) (width 0.2) (layer "B.Cu") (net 21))
 (segment (start 169.545 72.685) (end 117.475 72.685) (width 0.2) (layer "B.Cu") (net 21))
 (segment (start 172.085 70.145) (end 169.545 72.685) (width 0.2) (layer "B.Cu") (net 21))
 (segment (start 114.935 62.525) (end 118.745 62.525) (width 0.2) (layer "B.Cu") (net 22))
 (segment (start 133.985 62.525) (end 137.795 62.525) (width 0.2) (layer "B.Cu") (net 14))
 (segment (start 153.035 62.525) (end 156.845 62.525) (width 0.2) (layer "B.Cu") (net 16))
 (segment (start 175.895 62.525) (end 172.085 62.525) (width 0.2) (layer "B.Cu") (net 24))
 (segment (start 192.405 72.685) (end 191.147765 72.685) (width 0.2) (layer "F.Cu") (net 11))
 (segment (start 196.46 76.74) (end 196.46 68.5925) (width 0.2) (layer "F.Cu") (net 18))
 (segment (start 205.105 85.385) (end 196.46 76.74) (width 0.2) (layer "F.Cu") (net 18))
 (segment (start 202.565 80.305) (end 205.105 82.845) (width 0.2) (layer "F.Cu") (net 17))
 (segment (start 200.66 60.0925) (end 201.0625 60.0925) (width 0.2) (layer "F.Cu") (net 17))
 (segment (start 201.0625 60.0925) (end 202.565 61.595) (width 0.2) (layer "F.Cu") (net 17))
 (segment (start 202.565 61.595) (end 202.565 80.305) (width 0.2) (layer "F.Cu") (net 17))
 (segment (start 206.375 61.255) (end 206.375 58.42) (width 0.2) (layer "B.Cu") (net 15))
 (segment (start 205.105 62.525) (end 206.375 61.255) (width 0.2) (layer "B.Cu") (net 15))
 (segment (start 206.375 58.42) (end 204.13 56.175) (width 0.2) (layer "B.Cu") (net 15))
 (segment (start 163.195 59.985) (end 144.145 59.985) (width 0.2) (layer "B.Cu") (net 15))
 (segment (start 144.145 59.985) (end 125.095 59.985) (width 0.2) (layer "B.Cu") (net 15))
 (segment (start 204.13 56.175) (end 167.005 56.175) (width 0.2) (layer "B.Cu") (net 15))
 (segment (start 167.005 56.175) (end 163.195 59.985) (width 0.2) (layer "B.Cu") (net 15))
 (segment (start 179.705 57.445) (end 108.585 57.445) (width 0.2) (layer "F.Cu") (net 4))
 (segment (start 182.245 59.985) (end 179.705 57.445) (width 0.2) (layer "F.Cu") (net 4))
 (segment (start 108.585 57.445) (end 106.045 59.985) (width 0.2) (layer "F.Cu") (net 4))
 (segment (start 189.865 59.985) (end 192.405 62.525) (width 0.2) (layer "B.Cu") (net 4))
 (segment (start 86.995 59.985) (end 106.045 59.985) (width 0.2) (layer "B.Cu") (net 4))
 (segment (start 182.245 59.985) (end 189.865 59.985) (width 0.2) (layer "B.Cu") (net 4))
 (segment (start 192.405 65.065) (end 191.135 65.065) (width 0.2) (layer "B.Cu") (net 8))
 (segment (start 192.405 67.605) (end 191.875435 67.075435) (width 0.2) (layer "B.Cu") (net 9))
 (segment (start 192.405 67.206935) (end 192.405 67.605) (width 0.2) (layer "B.Cu") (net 9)))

